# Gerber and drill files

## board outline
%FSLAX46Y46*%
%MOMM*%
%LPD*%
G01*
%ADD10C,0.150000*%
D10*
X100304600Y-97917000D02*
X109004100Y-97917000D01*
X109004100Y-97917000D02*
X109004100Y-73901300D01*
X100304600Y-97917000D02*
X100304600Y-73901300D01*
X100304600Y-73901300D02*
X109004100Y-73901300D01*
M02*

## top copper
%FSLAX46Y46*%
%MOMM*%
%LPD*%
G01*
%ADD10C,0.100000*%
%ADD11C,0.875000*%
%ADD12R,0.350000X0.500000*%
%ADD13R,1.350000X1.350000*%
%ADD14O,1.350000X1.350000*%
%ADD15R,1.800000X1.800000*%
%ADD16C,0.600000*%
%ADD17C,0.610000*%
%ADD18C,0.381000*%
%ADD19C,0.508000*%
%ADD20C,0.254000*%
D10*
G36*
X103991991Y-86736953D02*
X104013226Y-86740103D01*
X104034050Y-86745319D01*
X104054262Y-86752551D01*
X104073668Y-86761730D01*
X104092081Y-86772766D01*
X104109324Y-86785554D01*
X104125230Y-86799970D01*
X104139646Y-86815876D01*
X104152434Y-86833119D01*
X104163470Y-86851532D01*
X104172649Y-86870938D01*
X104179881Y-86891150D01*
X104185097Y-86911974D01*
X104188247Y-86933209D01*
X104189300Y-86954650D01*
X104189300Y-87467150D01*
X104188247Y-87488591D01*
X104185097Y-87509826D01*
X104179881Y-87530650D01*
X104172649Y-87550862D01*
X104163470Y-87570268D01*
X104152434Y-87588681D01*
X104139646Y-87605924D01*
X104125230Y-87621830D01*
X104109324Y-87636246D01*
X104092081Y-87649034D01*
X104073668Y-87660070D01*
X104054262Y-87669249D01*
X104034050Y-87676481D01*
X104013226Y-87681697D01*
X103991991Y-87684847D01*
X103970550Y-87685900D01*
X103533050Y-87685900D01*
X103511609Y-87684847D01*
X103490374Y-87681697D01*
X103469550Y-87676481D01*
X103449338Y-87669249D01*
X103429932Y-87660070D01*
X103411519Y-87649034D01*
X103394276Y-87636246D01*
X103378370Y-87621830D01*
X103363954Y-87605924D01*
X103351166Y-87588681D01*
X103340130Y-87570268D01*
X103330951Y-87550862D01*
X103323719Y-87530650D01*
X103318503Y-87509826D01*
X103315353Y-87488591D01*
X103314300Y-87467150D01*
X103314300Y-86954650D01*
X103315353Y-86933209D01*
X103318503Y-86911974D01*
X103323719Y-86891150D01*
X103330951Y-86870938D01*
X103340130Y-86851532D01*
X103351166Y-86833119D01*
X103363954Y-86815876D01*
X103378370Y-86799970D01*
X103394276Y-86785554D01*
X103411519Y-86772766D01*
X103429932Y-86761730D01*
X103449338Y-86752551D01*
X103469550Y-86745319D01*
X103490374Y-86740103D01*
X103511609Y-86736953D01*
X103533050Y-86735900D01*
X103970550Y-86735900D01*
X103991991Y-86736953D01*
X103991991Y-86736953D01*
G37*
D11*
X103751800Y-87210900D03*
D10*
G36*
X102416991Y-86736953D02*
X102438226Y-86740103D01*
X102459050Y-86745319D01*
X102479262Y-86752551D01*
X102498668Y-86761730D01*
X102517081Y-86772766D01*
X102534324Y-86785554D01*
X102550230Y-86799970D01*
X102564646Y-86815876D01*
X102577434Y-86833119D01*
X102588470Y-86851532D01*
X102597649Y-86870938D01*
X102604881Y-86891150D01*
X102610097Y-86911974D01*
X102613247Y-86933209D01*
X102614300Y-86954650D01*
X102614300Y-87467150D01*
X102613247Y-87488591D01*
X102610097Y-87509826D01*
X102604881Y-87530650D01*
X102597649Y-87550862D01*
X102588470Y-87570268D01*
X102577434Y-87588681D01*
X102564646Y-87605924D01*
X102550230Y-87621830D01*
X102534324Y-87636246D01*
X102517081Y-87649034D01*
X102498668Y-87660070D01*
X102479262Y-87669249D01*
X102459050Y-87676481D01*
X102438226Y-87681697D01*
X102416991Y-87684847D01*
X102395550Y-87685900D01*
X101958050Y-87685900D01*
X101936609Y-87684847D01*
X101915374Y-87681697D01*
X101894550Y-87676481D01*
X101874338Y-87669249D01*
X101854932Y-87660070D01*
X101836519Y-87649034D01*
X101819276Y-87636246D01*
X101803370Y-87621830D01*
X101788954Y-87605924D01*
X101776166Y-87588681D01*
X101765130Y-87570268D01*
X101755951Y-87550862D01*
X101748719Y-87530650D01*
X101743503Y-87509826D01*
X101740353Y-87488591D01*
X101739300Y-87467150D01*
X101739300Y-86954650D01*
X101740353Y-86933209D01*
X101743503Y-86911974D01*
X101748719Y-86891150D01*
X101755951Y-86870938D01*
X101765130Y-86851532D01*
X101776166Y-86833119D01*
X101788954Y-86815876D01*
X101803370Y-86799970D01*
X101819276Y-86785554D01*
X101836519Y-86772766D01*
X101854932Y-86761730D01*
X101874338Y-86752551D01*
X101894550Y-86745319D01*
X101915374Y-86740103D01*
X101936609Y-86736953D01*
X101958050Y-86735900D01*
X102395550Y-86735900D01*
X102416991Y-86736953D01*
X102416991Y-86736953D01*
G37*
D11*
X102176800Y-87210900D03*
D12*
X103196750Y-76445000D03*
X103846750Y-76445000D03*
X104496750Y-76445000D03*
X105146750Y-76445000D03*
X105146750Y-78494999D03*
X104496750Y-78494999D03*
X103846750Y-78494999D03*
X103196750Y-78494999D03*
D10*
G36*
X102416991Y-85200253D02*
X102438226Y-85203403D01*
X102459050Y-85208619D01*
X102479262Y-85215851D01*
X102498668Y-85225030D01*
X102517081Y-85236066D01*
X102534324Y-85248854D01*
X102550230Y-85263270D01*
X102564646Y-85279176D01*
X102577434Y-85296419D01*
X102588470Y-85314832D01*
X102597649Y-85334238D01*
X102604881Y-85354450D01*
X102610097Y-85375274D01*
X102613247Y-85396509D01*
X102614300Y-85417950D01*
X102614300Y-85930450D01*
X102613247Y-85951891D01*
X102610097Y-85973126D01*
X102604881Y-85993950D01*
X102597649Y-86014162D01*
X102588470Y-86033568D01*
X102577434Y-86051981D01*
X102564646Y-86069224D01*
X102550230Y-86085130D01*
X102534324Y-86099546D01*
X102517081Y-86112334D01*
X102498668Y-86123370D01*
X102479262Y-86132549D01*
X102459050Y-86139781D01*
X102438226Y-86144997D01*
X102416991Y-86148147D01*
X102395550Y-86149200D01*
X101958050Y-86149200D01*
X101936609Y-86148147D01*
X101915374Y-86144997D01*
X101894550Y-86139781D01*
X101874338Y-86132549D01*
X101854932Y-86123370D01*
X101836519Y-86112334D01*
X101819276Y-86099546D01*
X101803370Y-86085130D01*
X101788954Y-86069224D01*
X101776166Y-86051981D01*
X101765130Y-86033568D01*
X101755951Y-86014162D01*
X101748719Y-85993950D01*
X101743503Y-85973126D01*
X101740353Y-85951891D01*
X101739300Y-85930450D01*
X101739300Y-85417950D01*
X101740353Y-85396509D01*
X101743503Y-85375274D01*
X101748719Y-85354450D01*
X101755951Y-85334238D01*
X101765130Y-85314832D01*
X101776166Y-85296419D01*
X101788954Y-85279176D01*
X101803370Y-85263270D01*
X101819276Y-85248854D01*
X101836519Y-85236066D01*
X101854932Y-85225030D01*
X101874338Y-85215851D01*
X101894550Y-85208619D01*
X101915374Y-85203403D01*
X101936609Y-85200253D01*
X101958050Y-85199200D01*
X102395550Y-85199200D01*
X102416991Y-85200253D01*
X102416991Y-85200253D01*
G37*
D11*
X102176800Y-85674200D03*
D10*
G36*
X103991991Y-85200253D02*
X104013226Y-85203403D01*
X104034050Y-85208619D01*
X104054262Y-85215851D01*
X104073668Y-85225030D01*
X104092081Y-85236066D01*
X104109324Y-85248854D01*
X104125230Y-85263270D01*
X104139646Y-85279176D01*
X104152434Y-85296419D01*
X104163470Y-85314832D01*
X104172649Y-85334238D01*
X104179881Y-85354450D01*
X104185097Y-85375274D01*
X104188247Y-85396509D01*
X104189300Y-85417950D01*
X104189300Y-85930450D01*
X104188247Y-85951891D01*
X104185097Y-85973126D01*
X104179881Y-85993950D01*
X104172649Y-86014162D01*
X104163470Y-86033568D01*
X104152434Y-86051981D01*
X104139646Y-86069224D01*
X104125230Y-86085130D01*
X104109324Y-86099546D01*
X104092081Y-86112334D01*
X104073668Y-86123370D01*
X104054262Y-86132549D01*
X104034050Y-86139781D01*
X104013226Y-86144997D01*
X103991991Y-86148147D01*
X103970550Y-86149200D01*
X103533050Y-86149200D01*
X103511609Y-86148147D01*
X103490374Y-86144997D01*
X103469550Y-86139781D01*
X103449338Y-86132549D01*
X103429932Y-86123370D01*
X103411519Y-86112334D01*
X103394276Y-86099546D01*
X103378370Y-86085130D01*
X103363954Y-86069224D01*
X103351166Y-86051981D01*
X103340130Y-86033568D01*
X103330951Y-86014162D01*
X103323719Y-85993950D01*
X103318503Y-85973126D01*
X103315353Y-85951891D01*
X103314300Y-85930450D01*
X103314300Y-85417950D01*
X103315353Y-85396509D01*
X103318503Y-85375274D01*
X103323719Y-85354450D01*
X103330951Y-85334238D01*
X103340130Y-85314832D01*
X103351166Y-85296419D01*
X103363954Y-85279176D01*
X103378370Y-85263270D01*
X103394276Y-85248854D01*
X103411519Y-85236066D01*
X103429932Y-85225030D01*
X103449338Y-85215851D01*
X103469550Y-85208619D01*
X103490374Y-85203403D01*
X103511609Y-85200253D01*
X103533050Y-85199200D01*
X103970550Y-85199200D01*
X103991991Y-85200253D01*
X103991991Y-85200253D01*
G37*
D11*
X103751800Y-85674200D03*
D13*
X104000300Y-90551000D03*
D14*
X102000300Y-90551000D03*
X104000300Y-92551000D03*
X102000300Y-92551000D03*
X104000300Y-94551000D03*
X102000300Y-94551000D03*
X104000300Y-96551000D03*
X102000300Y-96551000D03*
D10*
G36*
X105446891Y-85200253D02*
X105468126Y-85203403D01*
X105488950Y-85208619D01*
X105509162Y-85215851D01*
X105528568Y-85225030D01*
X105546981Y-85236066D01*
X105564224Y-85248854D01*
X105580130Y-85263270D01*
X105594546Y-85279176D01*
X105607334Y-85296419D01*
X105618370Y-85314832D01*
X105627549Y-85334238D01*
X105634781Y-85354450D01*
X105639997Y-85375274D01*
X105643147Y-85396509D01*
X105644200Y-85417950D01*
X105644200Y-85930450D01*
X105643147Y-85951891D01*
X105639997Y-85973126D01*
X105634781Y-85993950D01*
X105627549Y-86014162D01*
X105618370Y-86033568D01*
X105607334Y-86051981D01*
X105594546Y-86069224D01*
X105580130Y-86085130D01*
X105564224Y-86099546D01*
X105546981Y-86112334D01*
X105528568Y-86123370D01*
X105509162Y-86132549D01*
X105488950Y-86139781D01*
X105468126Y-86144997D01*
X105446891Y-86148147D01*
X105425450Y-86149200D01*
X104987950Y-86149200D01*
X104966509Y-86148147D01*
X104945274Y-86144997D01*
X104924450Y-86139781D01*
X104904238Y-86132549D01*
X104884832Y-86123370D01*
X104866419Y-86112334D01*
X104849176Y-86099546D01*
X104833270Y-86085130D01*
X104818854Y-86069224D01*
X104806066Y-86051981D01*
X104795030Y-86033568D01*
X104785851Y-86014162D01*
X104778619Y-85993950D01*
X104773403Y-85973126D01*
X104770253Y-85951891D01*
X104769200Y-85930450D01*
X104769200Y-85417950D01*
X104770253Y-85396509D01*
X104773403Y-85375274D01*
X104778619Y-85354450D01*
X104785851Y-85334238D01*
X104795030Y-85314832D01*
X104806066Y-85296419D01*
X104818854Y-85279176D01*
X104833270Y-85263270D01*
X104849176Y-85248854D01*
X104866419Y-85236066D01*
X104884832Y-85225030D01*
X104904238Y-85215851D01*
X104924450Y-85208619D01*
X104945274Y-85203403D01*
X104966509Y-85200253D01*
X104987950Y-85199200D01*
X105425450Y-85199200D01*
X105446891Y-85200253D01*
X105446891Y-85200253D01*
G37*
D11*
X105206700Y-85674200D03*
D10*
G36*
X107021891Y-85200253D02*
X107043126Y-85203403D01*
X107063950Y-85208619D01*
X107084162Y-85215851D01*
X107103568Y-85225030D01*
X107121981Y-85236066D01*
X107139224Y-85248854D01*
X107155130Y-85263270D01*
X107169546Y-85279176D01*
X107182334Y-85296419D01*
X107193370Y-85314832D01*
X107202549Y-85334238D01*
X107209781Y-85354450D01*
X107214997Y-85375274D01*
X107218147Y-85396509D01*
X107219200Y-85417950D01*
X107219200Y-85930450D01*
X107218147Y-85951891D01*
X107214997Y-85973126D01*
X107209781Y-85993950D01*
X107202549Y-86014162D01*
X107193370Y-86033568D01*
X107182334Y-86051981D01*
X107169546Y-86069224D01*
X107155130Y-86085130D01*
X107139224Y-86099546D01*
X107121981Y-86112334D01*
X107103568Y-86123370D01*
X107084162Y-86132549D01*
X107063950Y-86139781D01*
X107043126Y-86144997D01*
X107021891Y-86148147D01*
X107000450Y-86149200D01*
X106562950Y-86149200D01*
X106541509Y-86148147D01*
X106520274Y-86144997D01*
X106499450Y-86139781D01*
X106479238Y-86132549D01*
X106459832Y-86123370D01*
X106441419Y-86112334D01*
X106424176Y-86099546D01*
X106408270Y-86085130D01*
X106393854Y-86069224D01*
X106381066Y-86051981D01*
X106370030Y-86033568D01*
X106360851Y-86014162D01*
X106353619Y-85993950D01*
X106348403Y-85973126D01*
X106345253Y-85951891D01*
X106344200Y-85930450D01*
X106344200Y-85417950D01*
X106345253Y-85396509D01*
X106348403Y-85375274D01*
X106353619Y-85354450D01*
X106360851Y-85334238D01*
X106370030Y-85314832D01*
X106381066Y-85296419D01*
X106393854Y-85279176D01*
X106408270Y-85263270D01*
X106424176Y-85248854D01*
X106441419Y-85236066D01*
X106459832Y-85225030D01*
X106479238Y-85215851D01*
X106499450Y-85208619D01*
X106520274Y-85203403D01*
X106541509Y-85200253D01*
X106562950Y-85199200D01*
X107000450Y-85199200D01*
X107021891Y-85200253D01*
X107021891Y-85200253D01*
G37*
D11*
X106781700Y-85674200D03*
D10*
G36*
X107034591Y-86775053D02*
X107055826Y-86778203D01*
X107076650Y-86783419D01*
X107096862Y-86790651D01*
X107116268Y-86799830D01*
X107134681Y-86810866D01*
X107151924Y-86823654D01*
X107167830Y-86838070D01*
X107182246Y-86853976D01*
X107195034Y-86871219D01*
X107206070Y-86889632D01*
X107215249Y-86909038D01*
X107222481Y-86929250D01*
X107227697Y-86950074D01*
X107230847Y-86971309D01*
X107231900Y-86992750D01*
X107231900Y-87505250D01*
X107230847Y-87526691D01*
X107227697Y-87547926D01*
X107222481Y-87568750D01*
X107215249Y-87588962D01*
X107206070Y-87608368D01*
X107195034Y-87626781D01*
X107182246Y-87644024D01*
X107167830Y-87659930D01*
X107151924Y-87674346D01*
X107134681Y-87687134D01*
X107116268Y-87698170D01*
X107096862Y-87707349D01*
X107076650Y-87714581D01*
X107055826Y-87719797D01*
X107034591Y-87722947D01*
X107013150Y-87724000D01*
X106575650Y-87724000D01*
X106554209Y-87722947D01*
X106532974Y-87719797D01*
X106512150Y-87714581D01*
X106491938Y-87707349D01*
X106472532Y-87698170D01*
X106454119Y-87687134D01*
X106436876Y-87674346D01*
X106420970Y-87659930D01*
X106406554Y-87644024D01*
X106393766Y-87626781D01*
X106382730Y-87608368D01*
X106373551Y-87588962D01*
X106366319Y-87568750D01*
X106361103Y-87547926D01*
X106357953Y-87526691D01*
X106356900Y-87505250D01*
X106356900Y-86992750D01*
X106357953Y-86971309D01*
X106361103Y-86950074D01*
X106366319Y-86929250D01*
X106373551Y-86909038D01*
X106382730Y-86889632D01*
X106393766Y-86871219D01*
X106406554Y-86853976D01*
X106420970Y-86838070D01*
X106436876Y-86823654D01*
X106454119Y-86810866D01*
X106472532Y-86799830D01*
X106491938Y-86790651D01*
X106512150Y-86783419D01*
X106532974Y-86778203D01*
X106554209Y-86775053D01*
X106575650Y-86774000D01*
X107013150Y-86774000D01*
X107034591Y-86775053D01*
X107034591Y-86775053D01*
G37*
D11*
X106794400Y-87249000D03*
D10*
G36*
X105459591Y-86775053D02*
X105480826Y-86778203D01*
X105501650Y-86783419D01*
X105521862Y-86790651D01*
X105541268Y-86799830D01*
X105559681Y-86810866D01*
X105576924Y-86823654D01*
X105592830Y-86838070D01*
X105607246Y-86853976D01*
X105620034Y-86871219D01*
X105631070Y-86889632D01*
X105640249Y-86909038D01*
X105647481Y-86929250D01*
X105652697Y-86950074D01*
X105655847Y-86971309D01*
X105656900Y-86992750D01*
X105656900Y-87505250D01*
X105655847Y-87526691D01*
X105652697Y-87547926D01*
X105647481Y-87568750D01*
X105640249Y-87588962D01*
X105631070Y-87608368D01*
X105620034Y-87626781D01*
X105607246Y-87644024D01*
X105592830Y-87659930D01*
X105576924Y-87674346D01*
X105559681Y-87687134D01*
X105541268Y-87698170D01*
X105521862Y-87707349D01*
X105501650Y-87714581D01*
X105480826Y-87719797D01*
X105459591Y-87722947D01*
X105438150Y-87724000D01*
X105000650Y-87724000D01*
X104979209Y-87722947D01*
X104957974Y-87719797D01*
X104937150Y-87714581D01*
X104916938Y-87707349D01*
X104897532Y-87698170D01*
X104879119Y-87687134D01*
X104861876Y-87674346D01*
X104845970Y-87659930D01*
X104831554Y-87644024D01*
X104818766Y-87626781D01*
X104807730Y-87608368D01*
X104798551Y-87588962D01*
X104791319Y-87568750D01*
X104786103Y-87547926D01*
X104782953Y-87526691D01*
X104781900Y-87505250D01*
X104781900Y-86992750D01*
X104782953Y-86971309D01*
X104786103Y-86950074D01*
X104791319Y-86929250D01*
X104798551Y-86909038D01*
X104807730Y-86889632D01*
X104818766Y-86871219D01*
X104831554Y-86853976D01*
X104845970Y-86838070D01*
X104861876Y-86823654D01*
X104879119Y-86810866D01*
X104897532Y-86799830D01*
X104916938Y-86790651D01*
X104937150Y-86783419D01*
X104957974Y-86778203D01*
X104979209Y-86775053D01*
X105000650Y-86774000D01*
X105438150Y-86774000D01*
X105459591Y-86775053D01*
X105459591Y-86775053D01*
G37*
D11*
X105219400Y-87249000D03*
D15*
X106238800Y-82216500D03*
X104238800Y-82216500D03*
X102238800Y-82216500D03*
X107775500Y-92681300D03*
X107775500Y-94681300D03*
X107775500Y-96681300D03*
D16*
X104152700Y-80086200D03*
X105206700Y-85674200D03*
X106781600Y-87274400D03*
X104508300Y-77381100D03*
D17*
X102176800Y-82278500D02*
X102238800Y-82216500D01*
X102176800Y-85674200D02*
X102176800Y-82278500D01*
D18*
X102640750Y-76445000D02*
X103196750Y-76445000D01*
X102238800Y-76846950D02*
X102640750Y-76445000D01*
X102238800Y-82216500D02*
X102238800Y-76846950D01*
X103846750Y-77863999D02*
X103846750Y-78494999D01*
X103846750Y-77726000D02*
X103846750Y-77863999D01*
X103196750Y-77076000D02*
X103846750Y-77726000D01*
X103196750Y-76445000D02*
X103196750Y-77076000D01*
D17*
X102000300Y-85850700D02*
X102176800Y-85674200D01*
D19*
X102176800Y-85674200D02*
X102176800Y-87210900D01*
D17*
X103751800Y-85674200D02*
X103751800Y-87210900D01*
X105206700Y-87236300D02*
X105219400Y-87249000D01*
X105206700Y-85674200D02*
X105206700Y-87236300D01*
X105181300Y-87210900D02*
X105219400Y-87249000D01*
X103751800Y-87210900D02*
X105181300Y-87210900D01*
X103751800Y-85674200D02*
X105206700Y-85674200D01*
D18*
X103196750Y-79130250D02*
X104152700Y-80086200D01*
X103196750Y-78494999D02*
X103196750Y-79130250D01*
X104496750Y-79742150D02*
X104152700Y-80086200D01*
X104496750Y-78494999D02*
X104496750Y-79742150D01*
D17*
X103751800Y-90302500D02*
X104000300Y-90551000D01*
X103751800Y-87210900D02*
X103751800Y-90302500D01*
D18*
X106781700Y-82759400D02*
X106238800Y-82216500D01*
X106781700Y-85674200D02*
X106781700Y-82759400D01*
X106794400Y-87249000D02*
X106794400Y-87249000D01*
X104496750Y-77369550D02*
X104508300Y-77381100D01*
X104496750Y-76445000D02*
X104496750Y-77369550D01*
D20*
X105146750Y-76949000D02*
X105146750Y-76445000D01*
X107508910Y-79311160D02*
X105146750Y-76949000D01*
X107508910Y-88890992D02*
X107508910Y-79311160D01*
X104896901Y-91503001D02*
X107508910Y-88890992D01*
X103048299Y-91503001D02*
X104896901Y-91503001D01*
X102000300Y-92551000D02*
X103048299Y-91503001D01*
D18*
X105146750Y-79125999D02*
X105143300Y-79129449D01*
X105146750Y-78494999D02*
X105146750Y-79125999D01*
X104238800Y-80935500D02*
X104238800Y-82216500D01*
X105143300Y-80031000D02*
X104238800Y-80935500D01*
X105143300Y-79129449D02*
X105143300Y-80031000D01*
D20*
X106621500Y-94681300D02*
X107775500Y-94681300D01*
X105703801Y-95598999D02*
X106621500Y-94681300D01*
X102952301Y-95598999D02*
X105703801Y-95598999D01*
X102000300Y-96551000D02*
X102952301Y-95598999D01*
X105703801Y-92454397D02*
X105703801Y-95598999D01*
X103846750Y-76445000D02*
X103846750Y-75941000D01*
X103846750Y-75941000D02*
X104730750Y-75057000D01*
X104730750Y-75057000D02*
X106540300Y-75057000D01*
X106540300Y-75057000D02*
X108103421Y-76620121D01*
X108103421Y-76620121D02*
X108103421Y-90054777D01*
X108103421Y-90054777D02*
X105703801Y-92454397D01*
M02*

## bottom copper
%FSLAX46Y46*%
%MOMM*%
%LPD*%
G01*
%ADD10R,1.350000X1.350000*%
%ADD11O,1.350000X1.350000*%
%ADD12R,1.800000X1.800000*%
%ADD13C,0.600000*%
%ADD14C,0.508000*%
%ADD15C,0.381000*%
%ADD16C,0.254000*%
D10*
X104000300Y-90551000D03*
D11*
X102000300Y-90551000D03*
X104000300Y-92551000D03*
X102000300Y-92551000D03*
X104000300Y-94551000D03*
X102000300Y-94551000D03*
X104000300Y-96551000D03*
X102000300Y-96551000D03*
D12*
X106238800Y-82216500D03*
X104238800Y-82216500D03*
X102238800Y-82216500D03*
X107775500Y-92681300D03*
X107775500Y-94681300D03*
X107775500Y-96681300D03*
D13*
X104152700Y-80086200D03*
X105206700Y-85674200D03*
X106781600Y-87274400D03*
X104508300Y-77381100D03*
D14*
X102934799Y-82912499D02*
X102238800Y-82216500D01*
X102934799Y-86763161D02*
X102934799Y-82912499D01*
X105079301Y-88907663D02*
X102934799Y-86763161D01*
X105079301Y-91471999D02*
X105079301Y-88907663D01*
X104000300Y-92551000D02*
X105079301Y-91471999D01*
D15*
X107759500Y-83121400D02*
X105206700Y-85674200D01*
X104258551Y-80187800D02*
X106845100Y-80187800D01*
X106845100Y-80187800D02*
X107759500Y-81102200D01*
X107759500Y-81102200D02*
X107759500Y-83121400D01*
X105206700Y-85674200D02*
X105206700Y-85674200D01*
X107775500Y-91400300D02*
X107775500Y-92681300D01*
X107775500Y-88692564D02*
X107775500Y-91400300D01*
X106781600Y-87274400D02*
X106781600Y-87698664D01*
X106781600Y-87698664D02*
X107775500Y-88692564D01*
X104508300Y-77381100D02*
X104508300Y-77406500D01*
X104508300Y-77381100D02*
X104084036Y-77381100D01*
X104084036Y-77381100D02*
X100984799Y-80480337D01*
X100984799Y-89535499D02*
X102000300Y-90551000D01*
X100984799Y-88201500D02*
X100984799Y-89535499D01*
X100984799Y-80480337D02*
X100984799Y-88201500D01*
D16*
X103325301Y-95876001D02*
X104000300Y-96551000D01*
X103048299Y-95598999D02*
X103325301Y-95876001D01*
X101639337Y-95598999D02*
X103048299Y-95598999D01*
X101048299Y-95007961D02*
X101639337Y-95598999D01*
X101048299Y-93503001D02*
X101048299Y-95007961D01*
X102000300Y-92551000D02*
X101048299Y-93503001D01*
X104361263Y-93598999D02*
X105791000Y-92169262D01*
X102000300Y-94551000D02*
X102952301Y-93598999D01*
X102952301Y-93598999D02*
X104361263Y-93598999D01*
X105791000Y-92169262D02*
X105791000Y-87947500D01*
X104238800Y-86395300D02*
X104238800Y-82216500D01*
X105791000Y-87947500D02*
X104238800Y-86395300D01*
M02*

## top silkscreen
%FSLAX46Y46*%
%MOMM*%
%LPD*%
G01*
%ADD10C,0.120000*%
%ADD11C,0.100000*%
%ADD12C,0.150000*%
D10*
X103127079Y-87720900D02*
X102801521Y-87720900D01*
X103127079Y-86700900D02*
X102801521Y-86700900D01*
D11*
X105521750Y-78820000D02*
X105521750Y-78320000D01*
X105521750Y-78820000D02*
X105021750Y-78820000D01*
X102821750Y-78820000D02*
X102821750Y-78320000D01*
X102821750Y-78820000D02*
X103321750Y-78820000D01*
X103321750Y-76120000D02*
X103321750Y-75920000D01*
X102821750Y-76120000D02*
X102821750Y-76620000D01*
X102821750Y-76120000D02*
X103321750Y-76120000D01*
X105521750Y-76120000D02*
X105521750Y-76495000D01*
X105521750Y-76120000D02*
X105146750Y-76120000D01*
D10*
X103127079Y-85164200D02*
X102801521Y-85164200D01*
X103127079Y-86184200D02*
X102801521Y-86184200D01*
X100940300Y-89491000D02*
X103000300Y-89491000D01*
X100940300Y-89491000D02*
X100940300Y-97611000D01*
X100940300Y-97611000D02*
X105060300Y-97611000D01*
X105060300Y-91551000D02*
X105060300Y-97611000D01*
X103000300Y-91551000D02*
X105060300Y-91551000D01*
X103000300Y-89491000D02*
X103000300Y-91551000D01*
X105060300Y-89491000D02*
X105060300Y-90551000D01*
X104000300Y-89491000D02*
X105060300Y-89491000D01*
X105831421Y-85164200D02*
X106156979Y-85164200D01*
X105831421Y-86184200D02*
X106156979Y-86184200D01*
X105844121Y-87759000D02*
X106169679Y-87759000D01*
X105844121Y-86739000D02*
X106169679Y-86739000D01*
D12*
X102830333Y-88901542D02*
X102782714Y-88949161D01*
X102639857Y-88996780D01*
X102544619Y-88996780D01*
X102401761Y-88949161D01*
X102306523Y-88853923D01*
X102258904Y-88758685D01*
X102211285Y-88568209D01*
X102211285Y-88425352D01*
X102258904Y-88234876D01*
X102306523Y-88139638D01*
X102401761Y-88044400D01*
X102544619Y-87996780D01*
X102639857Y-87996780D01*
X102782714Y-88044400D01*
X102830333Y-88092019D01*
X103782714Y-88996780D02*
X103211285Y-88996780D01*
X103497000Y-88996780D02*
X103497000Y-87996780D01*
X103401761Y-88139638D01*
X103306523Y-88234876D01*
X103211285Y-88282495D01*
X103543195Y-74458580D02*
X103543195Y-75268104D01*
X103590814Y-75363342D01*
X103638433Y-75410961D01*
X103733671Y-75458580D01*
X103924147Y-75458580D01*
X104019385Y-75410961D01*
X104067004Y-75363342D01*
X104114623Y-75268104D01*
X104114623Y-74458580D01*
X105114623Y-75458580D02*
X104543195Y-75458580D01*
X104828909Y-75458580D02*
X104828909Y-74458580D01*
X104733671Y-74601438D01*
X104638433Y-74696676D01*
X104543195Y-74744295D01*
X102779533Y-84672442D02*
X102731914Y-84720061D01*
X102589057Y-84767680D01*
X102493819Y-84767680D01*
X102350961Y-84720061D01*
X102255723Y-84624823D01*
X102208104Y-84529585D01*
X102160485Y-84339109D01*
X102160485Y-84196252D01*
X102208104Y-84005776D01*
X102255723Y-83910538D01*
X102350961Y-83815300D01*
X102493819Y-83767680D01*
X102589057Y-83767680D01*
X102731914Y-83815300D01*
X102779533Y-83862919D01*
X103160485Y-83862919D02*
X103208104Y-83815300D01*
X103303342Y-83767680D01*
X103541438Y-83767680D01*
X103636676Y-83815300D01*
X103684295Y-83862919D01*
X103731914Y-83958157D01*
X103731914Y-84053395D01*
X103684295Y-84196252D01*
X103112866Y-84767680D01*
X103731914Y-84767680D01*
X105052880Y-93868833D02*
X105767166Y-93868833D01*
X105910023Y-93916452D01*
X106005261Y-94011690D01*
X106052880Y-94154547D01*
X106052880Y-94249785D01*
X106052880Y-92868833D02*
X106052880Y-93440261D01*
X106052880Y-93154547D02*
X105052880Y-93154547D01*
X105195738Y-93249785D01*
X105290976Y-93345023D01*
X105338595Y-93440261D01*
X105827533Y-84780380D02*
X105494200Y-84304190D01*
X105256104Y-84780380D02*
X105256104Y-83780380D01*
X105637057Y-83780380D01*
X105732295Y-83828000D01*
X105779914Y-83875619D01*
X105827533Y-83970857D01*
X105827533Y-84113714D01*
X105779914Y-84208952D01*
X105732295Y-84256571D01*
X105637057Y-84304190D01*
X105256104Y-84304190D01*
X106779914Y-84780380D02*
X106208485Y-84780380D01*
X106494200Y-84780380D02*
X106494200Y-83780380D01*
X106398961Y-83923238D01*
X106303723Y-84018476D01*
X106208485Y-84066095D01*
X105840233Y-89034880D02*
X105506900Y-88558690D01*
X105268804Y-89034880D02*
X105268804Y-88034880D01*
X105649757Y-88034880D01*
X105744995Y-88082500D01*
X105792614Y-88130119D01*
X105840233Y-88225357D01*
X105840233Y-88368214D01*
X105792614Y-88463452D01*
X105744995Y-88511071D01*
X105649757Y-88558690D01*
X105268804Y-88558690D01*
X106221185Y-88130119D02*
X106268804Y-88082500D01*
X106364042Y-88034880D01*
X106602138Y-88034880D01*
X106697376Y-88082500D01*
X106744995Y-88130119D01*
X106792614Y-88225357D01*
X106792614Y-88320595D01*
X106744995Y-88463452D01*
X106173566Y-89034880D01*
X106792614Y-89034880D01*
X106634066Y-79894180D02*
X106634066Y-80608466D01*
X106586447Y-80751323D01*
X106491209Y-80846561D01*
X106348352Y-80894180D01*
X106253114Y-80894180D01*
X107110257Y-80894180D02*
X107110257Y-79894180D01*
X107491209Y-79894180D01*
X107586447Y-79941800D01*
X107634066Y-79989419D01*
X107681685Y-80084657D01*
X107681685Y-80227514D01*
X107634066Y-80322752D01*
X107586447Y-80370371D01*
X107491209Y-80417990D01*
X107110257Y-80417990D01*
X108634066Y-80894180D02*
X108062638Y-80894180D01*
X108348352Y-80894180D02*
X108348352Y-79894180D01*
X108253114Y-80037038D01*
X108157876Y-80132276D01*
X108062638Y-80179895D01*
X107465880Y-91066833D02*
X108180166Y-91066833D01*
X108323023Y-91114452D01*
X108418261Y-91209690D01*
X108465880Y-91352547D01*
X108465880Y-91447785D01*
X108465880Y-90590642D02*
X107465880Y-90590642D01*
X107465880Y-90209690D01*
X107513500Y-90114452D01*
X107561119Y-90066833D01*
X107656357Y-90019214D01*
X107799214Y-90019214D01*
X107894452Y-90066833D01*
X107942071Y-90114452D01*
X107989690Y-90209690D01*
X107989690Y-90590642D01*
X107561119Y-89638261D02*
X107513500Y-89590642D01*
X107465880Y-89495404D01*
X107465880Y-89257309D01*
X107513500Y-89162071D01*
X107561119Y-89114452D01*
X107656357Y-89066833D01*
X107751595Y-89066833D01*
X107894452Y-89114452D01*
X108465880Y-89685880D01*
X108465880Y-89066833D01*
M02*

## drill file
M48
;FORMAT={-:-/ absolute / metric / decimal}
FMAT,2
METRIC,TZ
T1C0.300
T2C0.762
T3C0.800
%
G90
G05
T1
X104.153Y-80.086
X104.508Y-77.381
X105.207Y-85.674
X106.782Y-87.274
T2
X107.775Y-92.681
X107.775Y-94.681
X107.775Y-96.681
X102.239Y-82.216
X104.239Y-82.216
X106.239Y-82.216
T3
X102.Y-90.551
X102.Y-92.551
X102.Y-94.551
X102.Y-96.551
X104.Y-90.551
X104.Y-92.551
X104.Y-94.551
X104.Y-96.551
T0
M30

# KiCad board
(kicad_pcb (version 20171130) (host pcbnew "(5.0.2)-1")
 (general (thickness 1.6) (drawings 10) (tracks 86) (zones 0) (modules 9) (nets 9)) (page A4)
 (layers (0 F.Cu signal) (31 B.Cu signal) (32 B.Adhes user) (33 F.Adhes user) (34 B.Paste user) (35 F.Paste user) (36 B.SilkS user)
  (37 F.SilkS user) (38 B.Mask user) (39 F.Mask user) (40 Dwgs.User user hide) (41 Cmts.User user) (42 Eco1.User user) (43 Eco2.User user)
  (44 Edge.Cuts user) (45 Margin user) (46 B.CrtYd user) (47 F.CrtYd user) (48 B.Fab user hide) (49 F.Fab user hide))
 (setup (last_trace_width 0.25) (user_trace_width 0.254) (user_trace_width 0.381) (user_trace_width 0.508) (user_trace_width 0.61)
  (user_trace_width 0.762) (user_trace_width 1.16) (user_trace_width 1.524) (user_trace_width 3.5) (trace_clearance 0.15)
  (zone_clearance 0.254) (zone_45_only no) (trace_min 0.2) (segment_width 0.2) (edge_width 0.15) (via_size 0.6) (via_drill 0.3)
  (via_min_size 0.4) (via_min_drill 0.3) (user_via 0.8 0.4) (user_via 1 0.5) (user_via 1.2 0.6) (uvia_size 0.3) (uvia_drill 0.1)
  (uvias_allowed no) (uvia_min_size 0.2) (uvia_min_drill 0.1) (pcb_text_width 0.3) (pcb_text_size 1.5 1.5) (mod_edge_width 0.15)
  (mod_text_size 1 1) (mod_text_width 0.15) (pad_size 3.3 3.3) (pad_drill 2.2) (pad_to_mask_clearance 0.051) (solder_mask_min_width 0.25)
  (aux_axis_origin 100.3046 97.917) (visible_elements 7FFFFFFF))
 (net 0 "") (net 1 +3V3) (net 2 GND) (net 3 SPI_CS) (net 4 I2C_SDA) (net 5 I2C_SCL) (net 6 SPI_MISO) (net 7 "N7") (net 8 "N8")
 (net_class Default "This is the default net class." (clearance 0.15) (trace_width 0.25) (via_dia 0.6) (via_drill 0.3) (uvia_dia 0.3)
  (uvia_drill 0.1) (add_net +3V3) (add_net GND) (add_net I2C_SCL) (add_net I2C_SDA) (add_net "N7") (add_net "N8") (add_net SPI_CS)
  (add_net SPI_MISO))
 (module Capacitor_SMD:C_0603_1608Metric (layer F.Cu) (at 102.9643 87.2109 180)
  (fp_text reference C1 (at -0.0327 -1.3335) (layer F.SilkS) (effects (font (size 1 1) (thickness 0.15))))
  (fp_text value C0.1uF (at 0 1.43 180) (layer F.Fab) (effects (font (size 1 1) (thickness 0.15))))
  (fp_line (start -0.162779 -0.51) (end 0.162779 -0.51) (layer F.SilkS) (width 0.12))
  (fp_line (start -0.162779 0.51) (end 0.162779 0.51) (layer F.SilkS) (width 0.12))
  (pad 1 smd roundrect (at -0.7875 0 180) (size 0.875 0.95) (layers F.Cu F.Paste F.Mask) (roundrect_rratio 0.25) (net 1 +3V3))
  (pad 2 smd roundrect (at 0.7875 0 180) (size 0.875 0.95) (layers F.Cu F.Paste F.Mask) (roundrect_rratio 0.25) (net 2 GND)))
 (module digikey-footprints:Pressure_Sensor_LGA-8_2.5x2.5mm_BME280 (layer F.Cu) (at 104.17175 77.47)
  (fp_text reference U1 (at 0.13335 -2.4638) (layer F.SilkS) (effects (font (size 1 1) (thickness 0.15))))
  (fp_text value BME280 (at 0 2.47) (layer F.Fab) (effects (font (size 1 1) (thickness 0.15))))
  (fp_line (start 1.35 1.35) (end 1.35 0.85) (layer F.SilkS) (width 0.1))
  (fp_line (start 1.35 1.35) (end 0.85 1.35) (layer F.SilkS) (width 0.1))
  (fp_line (start -1.35 1.35) (end -1.35 0.85) (layer F.SilkS) (width 0.1))
  (fp_line (start -1.35 1.35) (end -0.85 1.35) (layer F.SilkS) (width 0.1))
  (fp_line (start -0.85 -1.35) (end -0.85 -1.55) (layer F.SilkS) (width 0.1))
  (fp_line (start -1.35 -1.35) (end -1.35 -0.85) (layer F.SilkS) (width 0.1))
  (fp_line (start -1.35 -1.35) (end -0.85 -1.35) (layer F.SilkS) (width 0.1))
  (fp_line (start 1.35 -1.35) (end 1.35 -0.975) (layer F.SilkS) (width 0.1))
  (fp_line (start 1.35 -1.35) (end 0.975 -1.35) (layer F.SilkS) (width 0.1))
  (pad 1 smd rect (at -0.975 -1.025) (size 0.35 0.5) (layers F.Cu F.Paste F.Mask) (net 2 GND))
  (pad 2 smd rect (at -0.325 -1.025) (size 0.35 0.5) (layers F.Cu F.Paste F.Mask) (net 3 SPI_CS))
  (pad 3 smd rect (at 0.325 -1.025) (size 0.35 0.5) (layers F.Cu F.Paste F.Mask) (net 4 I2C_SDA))
  (pad 4 smd rect (at 0.975 -1.025) (size 0.35 0.5) (layers F.Cu F.Paste F.Mask) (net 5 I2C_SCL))
  (pad 5 smd rect (at 0.975 1.024999) (size 0.35 0.5) (layers F.Cu F.Paste F.Mask) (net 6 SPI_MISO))
  (pad 6 smd rect (at 0.325 1.024999) (size 0.35 0.5) (layers F.Cu F.Paste F.Mask) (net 1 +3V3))
  (pad 7 smd rect (at -0.325 1.024999) (size 0.35 0.5) (layers F.Cu F.Paste F.Mask) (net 2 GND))
  (pad 8 smd rect (at -0.975 1.024999) (size 0.35 0.5) (layers F.Cu F.Paste F.Mask) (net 1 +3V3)))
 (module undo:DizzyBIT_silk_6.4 (layer B.Cu) (at 104.648 76.2635 180)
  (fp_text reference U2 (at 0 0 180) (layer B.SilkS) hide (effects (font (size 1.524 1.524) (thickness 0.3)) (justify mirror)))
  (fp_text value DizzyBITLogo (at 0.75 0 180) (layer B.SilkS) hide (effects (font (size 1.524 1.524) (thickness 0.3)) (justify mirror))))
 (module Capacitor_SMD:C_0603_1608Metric (layer F.Cu) (at 102.9643 85.6742 180)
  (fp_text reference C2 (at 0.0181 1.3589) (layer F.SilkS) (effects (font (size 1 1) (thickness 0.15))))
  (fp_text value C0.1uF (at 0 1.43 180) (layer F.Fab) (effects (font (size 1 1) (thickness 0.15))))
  (fp_line (start -0.162779 0.51) (end 0.162779 0.51) (layer F.SilkS) (width 0.12))
  (fp_line (start -0.162779 -0.51) (end 0.162779 -0.51) (layer F.SilkS) (width 0.12))
  (pad 2 smd roundrect (at 0.7875 0 180) (size 0.875 0.95) (layers F.Cu F.Paste F.Mask) (roundrect_rratio 0.25) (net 2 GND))
  (pad 1 smd roundrect (at -0.7875 0 180) (size 0.875 0.95) (layers F.Cu F.Paste F.Mask) (roundrect_rratio 0.25) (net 1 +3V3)))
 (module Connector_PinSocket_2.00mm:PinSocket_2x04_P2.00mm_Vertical (layer F.Cu) (at 104.0003 90.551)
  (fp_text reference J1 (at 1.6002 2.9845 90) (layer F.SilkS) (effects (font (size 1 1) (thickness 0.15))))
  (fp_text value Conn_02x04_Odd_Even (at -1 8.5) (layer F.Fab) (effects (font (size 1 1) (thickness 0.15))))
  (fp_line (start -3.06 -1.06) (end -1 -1.06) (layer F.SilkS) (width 0.12))
  (fp_line (start -3.06 -1.06) (end -3.06 7.06) (layer F.SilkS) (width 0.12))
  (fp_line (start -3.06 7.06) (end 1.06 7.06) (layer F.SilkS) (width 0.12))
  (fp_line (start 1.06 1) (end 1.06 7.06) (layer F.SilkS) (width 0.12))
  (fp_line (start -1 1) (end 1.06 1) (layer F.SilkS) (width 0.12))
  (fp_line (start -1 -1.06) (end -1 1) (layer F.SilkS) (width 0.12))
  (fp_line (start 1.06 -1.06) (end 1.06 0) (layer F.SilkS) (width 0.12))
  (fp_line (start 0 -1.06) (end 1.06 -1.06) (layer F.SilkS) (width 0.12))
  (pad 1 thru_hole rect (at 0 0) (size 1.35 1.35) (drill 0.8) (layers *.Cu *.Mask) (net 1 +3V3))
  (pad 2 thru_hole oval (at -2 0) (size 1.35 1.35) (drill 0.8) (layers *.Cu *.Mask) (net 4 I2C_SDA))
  (pad 3 thru_hole oval (at 0 2) (size 1.35 1.35) (drill 0.8) (layers *.Cu *.Mask) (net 2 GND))
  (pad 4 thru_hole oval (at -2 2) (size 1.35 1.35) (drill 0.8) (layers *.Cu *.Mask) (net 5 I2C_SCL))
  (pad 5 thru_hole oval (at 0 4) (size 1.35 1.35) (drill 0.8) (layers *.Cu *.Mask))
  (pad 6 thru_hole oval (at -2 4) (size 1.35 1.35) (drill 0.8) (layers *.Cu *.Mask) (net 6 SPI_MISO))
  (pad 7 thru_hole oval (at 0 6) (size 1.35 1.35) (drill 0.8) (layers *.Cu *.Mask) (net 5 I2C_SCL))
  (pad 8 thru_hole oval (at -2 6) (size 1.35 1.35) (drill 0.8) (layers *.Cu *.Mask) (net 3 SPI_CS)))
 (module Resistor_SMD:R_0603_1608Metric (layer F.Cu) (at 105.9942 85.6742)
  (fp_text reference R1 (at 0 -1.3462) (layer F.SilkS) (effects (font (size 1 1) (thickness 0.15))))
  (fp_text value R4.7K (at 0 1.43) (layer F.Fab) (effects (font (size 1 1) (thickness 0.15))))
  (fp_line (start -0.162779 -0.51) (end 0.162779 -0.51) (layer F.SilkS) (width 0.12))
  (fp_line (start -0.162779 0.51) (end 0.162779 0.51) (layer F.SilkS) (width 0.12))
  (pad 1 smd roundrect (at -0.7875 0) (size 0.875 0.95) (layers F.Cu F.Paste F.Mask) (roundrect_rratio 0.25) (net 1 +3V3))
  (pad 2 smd roundrect (at 0.7875 0) (size 0.875 0.95) (layers F.Cu F.Paste F.Mask) (roundrect_rratio 0.25) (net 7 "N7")))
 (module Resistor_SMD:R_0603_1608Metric (layer F.Cu) (at 106.0069 87.249)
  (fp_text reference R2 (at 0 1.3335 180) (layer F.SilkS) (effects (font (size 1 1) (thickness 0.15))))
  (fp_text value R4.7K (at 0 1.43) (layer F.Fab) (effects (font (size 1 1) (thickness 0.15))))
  (fp_line (start -0.162779 0.51) (end 0.162779 0.51) (layer F.SilkS) (width 0.12))
  (fp_line (start -0.162779 -0.51) (end 0.162779 -0.51) (layer F.SilkS) (width 0.12))
  (pad 2 smd roundrect (at 0.7875 0) (size 0.875 0.95) (layers F.Cu F.Paste F.Mask) (roundrect_rratio 0.25) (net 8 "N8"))
  (pad 1 smd roundrect (at -0.7875 0) (size 0.875 0.95) (layers F.Cu F.Paste F.Mask) (roundrect_rratio 0.25) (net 1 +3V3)))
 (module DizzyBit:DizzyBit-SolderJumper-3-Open (layer B.Cu) (at 107.2388 81.2165 180)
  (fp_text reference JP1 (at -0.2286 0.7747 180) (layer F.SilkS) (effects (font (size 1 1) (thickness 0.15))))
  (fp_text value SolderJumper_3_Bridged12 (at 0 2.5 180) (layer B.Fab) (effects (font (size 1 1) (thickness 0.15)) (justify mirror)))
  (pad 1 thru_hole rect (at 1 -1) (size 1.8 1.8) (drill 0.762) (layers *.Cu *.Mask) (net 7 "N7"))
  (pad 2 thru_hole rect (at 3 -1 180) (size 1.8 1.8) (drill 0.762) (layers *.Cu *.Mask) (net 6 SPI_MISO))
  (pad 3 thru_hole rect (at 5 -1 180) (size 1.8 1.8) (drill 0.762) (layers *.Cu *.Mask) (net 2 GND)))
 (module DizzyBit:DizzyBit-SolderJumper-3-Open (layer F.Cu) (at 108.7755 91.6813 270)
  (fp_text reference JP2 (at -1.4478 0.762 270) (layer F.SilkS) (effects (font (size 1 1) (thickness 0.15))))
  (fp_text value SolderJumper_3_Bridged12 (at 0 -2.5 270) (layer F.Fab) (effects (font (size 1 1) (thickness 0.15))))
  (pad 1 thru_hole rect (at 1 1 90) (size 1.8 1.8) (drill 0.762) (layers *.Cu *.Mask) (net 8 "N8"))
  (pad 2 thru_hole rect (at 3 1 270) (size 1.8 1.8) (drill 0.762) (layers *.Cu *.Mask) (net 3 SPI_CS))
  (pad 3 thru_hole rect (at 5 1 270) (size 1.8 1.8) (drill 0.762) (layers *.Cu *.Mask)))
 (gr_line (start 100.3046 97.917) (end 109.0041 97.917) (layer Edge.Cuts) (width 0.15))
 (gr_line (start 109.0041 97.917) (end 109.0041 73.9013) (layer Edge.Cuts) (width 0.15))
 (gr_line (start 100.3046 97.917) (end 100.3046 73.9013) (layer Edge.Cuts) (width 0.15))
 (gr_line (start 100.3046 73.9013) (end 109.0041 73.9013) (layer Edge.Cuts) (width 0.15))
 (segment (start 102.1768 82.2785) (end 102.2388 82.2165) (width 0.61) (layer F.Cu) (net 2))
 (segment (start 102.1768 85.6742) (end 102.1768 82.2785) (width 0.61) (layer F.Cu) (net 2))
 (segment (start 102.64075 76.445) (end 103.19675 76.445) (width 0.381) (layer F.Cu) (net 2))
 (segment (start 102.2388 76.84695) (end 102.64075 76.445) (width 0.381) (layer F.Cu) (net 2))
 (segment (start 102.2388 82.2165) (end 102.2388 76.84695) (width 0.381) (layer F.Cu) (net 2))
 (segment (start 103.84675 77.863999) (end 103.84675 78.494999) (width 0.381) (layer F.Cu) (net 2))
 (segment (start 103.84675 77.726) (end 103.84675 77.863999) (width 0.381) (layer F.Cu) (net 2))
 (segment (start 103.19675 77.076) (end 103.84675 77.726) (width 0.381) (layer F.Cu) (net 2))
 (segment (start 103.19675 76.445) (end 103.19675 77.076) (width 0.381) (layer F.Cu) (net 2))
 (segment (start 102.0003 85.8507) (end 102.1768 85.6742) (width 0.61) (layer F.Cu) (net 2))
 (segment (start 102.934799 82.912499) (end 102.2388 82.2165) (width 0.508) (layer B.Cu) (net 2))
 (segment (start 102.934799 86.763161) (end 102.934799 82.912499) (width 0.508) (layer B.Cu) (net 2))
 (segment (start 105.079301 88.907663) (end 102.934799 86.763161) (width 0.508) (layer B.Cu) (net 2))
 (segment (start 105.079301 91.471999) (end 105.079301 88.907663) (width 0.508) (layer B.Cu) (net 2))
 (segment (start 104.0003 92.551) (end 105.079301 91.471999) (width 0.508) (layer B.Cu) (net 2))
 (segment (start 102.1768 85.6742) (end 102.1768 87.2109) (width 0.508) (layer F.Cu) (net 2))
 (segment (start 107.7595 83.1214) (end 105.2067 85.6742) (width 0.381) (layer B.Cu) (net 1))
 (segment (start 104.258551 80.1878) (end 106.8451 80.1878) (width 0.381) (layer B.Cu) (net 1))
 (segment (start 106.8451 80.1878) (end 107.7595 81.1022) (width 0.381) (layer B.Cu) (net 1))
 (segment (start 107.7595 81.1022) (end 107.7595 83.1214) (width 0.381) (layer B.Cu) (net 1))
 (segment (start 103.7518 85.6742) (end 103.7518 87.2109) (width 0.61) (layer F.Cu) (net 1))
 (segment (start 105.2067 87.2363) (end 105.2194 87.249) (width 0.61) (layer F.Cu) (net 1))
 (segment (start 105.2067 85.6742) (end 105.2067 87.2363) (width 0.61) (layer F.Cu) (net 1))
 (segment (start 105.1813 87.2109) (end 105.2194 87.249) (width 0.61) (layer F.Cu) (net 1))
 (segment (start 103.7518 87.2109) (end 105.1813 87.2109) (width 0.61) (layer F.Cu) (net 1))
 (segment (start 103.7518 85.6742) (end 105.2067 85.6742) (width 0.61) (layer F.Cu) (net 1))
 (via (at 104.1527 80.0862) (size 0.6) (drill 0.3) (layers F.Cu B.Cu) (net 1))
 (segment (start 103.19675 79.13025) (end 104.1527 80.0862) (width 0.381) (layer F.Cu) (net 1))
 (segment (start 103.19675 78.494999) (end 103.19675 79.13025) (width 0.381) (layer F.Cu) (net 1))
 (segment (start 104.49675 79.74215) (end 104.1527 80.0862) (width 0.381) (layer F.Cu) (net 1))
 (segment (start 104.49675 78.494999) (end 104.49675 79.74215) (width 0.381) (layer F.Cu) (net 1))
 (segment (start 105.2067 85.6742) (end 105.2067 85.6742) (width 0.381) (layer B.Cu) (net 1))
 (via (at 105.2067 85.6742) (size 0.6) (drill 0.3) (layers F.Cu B.Cu) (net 1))
 (segment (start 103.7518 90.3025) (end 104.0003 90.551) (width 0.61) (layer F.Cu) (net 1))
 (segment (start 103.7518 87.2109) (end 103.7518 90.3025) (width 0.61) (layer F.Cu) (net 1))
 (segment (start 106.7817 82.7594) (end 106.2388 82.2165) (width 0.381) (layer F.Cu) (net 7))
 (segment (start 106.7817 85.6742) (end 106.7817 82.7594) (width 0.381) (layer F.Cu) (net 7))
 (segment (start 106.7944 87.249) (end 106.7944 87.249) (width 0.381) (layer F.Cu) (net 8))
 (via (at 106.7816 87.2744) (size 0.6) (drill 0.3) (layers F.Cu B.Cu) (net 8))
 (segment (start 107.7755 91.4003) (end 107.7755 92.6813) (width 0.381) (layer B.Cu) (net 8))
 (segment (start 107.7755 88.692564) (end 107.7755 91.4003) (width 0.381) (layer B.Cu) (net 8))
 (segment (start 106.7816 87.2744) (end 106.7816 87.698664) (width 0.381) (layer B.Cu) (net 8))
 (segment (start 106.7816 87.698664) (end 107.7755 88.692564) (width 0.381) (layer B.Cu) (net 8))
 (segment (start 104.5083 77.3811) (end 104.5083 77.4065) (width 0.381) (layer B.Cu) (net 4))
 (via (at 104.5083 77.3811) (size 0.6) (drill 0.3) (layers F.Cu B.Cu) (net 4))
 (segment (start 104.49675 77.36955) (end 104.5083 77.3811) (width 0.381) (layer F.Cu) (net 4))
 (segment (start 104.49675 76.445) (end 104.49675 77.36955) (width 0.381) (layer F.Cu) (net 4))
 (segment (start 104.5083 77.3811) (end 104.084036 77.3811) (width 0.381) (layer B.Cu) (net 4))
 (segment (start 104.084036 77.3811) (end 100.984799 80.480337) (width 0.381) (layer B.Cu) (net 4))
 (segment (start 100.984799 89.535499) (end 102.0003 90.551) (width 0.381) (layer B.Cu) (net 4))
 (segment (start 100.984799 88.2015) (end 100.984799 89.535499) (width 0.381) (layer B.Cu) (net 4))
 (segment (start 100.984799 80.480337) (end 100.984799 88.2015) (width 0.381) (layer B.Cu) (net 4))
 (segment (start 105.14675 76.949) (end 105.14675 76.445) (width 0.254) (layer F.Cu) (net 5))
 (segment (start 107.50891 79.31116) (end 105.14675 76.949) (width 0.254) (layer F.Cu) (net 5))
 (segment (start 107.50891 88.890992) (end 107.50891 79.31116) (width 0.254) (layer F.Cu) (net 5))
 (segment (start 104.896901 91.503001) (end 107.50891 88.890992) (width 0.254) (layer F.Cu) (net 5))
 (segment (start 103.048299 91.503001) (end 104.896901 91.503001) (width 0.254) (layer F.Cu) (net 5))
 (segment (start 102.0003 92.551) (end 103.048299 91.503001) (width 0.254) (layer F.Cu) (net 5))
 (segment (start 103.325301 95.876001) (end 104.0003 96.551) (width 0.254) (layer B.Cu) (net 5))
 (segment (start 103.048299 95.598999) (end 103.325301 95.876001) (width 0.254) (layer B.Cu) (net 5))
 (segment (start 101.639337 95.598999) (end 103.048299 95.598999) (width 0.254) (layer B.Cu) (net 5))
 (segment (start 101.048299 95.007961) (end 101.639337 95.598999) (width 0.254) (layer B.Cu) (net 5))
 (segment (start 101.048299 93.503001) (end 101.048299 95.007961) (width 0.254) (layer B.Cu) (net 5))
 (segment (start 102.0003 92.551) (end 101.048299 93.503001) (width 0.254) (layer B.Cu) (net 5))
 (segment (start 105.14675 79.125999) (end 105.1433 79.129449) (width 0.381) (layer F.Cu) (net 6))
 (segment (start 105.14675 78.494999) (end 105.14675 79.125999) (width 0.381) (layer F.Cu) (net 6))
 (segment (start 104.2388 80.9355) (end 104.2388 82.2165) (width 0.381) (layer F.Cu) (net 6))
 (segment (start 105.1433 80.031) (end 104.2388 80.9355) (width 0.381) (layer F.Cu) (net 6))
 (segment (start 105.1433 79.129449) (end 105.1433 80.031) (width 0.381) (layer F.Cu) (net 6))
 (segment (start 104.361263 93.598999) (end 105.791 92.169262) (width 0.254) (layer B.Cu) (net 6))
 (segment (start 102.0003 94.551) (end 102.952301 93.598999) (width 0.254) (layer B.Cu) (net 6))
 (segment (start 102.952301 93.598999) (end 104.361263 93.598999) (width 0.254) (layer B.Cu) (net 6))
 (segment (start 105.791 92.169262) (end 105.791 87.9475) (width 0.254) (layer B.Cu) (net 6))
 (segment (start 104.2388 86.3953) (end 104.2388 82.2165) (width 0.254) (layer B.Cu) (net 6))
 (segment (start 105.791 87.9475) (end 104.2388 86.3953) (width 0.254) (layer B.Cu) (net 6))
 (segment (start 106.6215 94.6813) (end 107.7755 94.6813) (width 0.254) (layer F.Cu) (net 3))
 (segment (start 105.703801 95.598999) (end 106.6215 94.6813) (width 0.254) (layer F.Cu) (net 3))
 (segment (start 102.952301 95.598999) (end 105.703801 95.598999) (width 0.254) (layer F.Cu) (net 3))
 (segment (start 102.0003 96.551) (end 102.952301 95.598999) (width 0.254) (layer F.Cu) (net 3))
 (segment (start 105.703801 92.454397) (end 105.703801 95.598999) (width 0.254) (layer F.Cu) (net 3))
 (segment (start 103.84675 76.445) (end 103.84675 75.941) (width 0.254) (layer F.Cu) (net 3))
 (segment (start 103.84675 75.941) (end 104.73075 75.057) (width 0.254) (layer F.Cu) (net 3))
 (segment (start 104.73075 75.057) (end 106.5403 75.057) (width 0.254) (layer F.Cu) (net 3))
 (segment (start 106.5403 75.057) (end 108.103421 76.620121) (width 0.254) (layer F.Cu) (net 3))
 (segment (start 108.103421 76.620121) (end 108.103421 90.054777) (width 0.254) (layer F.Cu) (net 3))
 (segment (start 108.103421 90.054777) (end 105.703801 92.454397) (width 0.254) (layer F.Cu) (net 3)))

